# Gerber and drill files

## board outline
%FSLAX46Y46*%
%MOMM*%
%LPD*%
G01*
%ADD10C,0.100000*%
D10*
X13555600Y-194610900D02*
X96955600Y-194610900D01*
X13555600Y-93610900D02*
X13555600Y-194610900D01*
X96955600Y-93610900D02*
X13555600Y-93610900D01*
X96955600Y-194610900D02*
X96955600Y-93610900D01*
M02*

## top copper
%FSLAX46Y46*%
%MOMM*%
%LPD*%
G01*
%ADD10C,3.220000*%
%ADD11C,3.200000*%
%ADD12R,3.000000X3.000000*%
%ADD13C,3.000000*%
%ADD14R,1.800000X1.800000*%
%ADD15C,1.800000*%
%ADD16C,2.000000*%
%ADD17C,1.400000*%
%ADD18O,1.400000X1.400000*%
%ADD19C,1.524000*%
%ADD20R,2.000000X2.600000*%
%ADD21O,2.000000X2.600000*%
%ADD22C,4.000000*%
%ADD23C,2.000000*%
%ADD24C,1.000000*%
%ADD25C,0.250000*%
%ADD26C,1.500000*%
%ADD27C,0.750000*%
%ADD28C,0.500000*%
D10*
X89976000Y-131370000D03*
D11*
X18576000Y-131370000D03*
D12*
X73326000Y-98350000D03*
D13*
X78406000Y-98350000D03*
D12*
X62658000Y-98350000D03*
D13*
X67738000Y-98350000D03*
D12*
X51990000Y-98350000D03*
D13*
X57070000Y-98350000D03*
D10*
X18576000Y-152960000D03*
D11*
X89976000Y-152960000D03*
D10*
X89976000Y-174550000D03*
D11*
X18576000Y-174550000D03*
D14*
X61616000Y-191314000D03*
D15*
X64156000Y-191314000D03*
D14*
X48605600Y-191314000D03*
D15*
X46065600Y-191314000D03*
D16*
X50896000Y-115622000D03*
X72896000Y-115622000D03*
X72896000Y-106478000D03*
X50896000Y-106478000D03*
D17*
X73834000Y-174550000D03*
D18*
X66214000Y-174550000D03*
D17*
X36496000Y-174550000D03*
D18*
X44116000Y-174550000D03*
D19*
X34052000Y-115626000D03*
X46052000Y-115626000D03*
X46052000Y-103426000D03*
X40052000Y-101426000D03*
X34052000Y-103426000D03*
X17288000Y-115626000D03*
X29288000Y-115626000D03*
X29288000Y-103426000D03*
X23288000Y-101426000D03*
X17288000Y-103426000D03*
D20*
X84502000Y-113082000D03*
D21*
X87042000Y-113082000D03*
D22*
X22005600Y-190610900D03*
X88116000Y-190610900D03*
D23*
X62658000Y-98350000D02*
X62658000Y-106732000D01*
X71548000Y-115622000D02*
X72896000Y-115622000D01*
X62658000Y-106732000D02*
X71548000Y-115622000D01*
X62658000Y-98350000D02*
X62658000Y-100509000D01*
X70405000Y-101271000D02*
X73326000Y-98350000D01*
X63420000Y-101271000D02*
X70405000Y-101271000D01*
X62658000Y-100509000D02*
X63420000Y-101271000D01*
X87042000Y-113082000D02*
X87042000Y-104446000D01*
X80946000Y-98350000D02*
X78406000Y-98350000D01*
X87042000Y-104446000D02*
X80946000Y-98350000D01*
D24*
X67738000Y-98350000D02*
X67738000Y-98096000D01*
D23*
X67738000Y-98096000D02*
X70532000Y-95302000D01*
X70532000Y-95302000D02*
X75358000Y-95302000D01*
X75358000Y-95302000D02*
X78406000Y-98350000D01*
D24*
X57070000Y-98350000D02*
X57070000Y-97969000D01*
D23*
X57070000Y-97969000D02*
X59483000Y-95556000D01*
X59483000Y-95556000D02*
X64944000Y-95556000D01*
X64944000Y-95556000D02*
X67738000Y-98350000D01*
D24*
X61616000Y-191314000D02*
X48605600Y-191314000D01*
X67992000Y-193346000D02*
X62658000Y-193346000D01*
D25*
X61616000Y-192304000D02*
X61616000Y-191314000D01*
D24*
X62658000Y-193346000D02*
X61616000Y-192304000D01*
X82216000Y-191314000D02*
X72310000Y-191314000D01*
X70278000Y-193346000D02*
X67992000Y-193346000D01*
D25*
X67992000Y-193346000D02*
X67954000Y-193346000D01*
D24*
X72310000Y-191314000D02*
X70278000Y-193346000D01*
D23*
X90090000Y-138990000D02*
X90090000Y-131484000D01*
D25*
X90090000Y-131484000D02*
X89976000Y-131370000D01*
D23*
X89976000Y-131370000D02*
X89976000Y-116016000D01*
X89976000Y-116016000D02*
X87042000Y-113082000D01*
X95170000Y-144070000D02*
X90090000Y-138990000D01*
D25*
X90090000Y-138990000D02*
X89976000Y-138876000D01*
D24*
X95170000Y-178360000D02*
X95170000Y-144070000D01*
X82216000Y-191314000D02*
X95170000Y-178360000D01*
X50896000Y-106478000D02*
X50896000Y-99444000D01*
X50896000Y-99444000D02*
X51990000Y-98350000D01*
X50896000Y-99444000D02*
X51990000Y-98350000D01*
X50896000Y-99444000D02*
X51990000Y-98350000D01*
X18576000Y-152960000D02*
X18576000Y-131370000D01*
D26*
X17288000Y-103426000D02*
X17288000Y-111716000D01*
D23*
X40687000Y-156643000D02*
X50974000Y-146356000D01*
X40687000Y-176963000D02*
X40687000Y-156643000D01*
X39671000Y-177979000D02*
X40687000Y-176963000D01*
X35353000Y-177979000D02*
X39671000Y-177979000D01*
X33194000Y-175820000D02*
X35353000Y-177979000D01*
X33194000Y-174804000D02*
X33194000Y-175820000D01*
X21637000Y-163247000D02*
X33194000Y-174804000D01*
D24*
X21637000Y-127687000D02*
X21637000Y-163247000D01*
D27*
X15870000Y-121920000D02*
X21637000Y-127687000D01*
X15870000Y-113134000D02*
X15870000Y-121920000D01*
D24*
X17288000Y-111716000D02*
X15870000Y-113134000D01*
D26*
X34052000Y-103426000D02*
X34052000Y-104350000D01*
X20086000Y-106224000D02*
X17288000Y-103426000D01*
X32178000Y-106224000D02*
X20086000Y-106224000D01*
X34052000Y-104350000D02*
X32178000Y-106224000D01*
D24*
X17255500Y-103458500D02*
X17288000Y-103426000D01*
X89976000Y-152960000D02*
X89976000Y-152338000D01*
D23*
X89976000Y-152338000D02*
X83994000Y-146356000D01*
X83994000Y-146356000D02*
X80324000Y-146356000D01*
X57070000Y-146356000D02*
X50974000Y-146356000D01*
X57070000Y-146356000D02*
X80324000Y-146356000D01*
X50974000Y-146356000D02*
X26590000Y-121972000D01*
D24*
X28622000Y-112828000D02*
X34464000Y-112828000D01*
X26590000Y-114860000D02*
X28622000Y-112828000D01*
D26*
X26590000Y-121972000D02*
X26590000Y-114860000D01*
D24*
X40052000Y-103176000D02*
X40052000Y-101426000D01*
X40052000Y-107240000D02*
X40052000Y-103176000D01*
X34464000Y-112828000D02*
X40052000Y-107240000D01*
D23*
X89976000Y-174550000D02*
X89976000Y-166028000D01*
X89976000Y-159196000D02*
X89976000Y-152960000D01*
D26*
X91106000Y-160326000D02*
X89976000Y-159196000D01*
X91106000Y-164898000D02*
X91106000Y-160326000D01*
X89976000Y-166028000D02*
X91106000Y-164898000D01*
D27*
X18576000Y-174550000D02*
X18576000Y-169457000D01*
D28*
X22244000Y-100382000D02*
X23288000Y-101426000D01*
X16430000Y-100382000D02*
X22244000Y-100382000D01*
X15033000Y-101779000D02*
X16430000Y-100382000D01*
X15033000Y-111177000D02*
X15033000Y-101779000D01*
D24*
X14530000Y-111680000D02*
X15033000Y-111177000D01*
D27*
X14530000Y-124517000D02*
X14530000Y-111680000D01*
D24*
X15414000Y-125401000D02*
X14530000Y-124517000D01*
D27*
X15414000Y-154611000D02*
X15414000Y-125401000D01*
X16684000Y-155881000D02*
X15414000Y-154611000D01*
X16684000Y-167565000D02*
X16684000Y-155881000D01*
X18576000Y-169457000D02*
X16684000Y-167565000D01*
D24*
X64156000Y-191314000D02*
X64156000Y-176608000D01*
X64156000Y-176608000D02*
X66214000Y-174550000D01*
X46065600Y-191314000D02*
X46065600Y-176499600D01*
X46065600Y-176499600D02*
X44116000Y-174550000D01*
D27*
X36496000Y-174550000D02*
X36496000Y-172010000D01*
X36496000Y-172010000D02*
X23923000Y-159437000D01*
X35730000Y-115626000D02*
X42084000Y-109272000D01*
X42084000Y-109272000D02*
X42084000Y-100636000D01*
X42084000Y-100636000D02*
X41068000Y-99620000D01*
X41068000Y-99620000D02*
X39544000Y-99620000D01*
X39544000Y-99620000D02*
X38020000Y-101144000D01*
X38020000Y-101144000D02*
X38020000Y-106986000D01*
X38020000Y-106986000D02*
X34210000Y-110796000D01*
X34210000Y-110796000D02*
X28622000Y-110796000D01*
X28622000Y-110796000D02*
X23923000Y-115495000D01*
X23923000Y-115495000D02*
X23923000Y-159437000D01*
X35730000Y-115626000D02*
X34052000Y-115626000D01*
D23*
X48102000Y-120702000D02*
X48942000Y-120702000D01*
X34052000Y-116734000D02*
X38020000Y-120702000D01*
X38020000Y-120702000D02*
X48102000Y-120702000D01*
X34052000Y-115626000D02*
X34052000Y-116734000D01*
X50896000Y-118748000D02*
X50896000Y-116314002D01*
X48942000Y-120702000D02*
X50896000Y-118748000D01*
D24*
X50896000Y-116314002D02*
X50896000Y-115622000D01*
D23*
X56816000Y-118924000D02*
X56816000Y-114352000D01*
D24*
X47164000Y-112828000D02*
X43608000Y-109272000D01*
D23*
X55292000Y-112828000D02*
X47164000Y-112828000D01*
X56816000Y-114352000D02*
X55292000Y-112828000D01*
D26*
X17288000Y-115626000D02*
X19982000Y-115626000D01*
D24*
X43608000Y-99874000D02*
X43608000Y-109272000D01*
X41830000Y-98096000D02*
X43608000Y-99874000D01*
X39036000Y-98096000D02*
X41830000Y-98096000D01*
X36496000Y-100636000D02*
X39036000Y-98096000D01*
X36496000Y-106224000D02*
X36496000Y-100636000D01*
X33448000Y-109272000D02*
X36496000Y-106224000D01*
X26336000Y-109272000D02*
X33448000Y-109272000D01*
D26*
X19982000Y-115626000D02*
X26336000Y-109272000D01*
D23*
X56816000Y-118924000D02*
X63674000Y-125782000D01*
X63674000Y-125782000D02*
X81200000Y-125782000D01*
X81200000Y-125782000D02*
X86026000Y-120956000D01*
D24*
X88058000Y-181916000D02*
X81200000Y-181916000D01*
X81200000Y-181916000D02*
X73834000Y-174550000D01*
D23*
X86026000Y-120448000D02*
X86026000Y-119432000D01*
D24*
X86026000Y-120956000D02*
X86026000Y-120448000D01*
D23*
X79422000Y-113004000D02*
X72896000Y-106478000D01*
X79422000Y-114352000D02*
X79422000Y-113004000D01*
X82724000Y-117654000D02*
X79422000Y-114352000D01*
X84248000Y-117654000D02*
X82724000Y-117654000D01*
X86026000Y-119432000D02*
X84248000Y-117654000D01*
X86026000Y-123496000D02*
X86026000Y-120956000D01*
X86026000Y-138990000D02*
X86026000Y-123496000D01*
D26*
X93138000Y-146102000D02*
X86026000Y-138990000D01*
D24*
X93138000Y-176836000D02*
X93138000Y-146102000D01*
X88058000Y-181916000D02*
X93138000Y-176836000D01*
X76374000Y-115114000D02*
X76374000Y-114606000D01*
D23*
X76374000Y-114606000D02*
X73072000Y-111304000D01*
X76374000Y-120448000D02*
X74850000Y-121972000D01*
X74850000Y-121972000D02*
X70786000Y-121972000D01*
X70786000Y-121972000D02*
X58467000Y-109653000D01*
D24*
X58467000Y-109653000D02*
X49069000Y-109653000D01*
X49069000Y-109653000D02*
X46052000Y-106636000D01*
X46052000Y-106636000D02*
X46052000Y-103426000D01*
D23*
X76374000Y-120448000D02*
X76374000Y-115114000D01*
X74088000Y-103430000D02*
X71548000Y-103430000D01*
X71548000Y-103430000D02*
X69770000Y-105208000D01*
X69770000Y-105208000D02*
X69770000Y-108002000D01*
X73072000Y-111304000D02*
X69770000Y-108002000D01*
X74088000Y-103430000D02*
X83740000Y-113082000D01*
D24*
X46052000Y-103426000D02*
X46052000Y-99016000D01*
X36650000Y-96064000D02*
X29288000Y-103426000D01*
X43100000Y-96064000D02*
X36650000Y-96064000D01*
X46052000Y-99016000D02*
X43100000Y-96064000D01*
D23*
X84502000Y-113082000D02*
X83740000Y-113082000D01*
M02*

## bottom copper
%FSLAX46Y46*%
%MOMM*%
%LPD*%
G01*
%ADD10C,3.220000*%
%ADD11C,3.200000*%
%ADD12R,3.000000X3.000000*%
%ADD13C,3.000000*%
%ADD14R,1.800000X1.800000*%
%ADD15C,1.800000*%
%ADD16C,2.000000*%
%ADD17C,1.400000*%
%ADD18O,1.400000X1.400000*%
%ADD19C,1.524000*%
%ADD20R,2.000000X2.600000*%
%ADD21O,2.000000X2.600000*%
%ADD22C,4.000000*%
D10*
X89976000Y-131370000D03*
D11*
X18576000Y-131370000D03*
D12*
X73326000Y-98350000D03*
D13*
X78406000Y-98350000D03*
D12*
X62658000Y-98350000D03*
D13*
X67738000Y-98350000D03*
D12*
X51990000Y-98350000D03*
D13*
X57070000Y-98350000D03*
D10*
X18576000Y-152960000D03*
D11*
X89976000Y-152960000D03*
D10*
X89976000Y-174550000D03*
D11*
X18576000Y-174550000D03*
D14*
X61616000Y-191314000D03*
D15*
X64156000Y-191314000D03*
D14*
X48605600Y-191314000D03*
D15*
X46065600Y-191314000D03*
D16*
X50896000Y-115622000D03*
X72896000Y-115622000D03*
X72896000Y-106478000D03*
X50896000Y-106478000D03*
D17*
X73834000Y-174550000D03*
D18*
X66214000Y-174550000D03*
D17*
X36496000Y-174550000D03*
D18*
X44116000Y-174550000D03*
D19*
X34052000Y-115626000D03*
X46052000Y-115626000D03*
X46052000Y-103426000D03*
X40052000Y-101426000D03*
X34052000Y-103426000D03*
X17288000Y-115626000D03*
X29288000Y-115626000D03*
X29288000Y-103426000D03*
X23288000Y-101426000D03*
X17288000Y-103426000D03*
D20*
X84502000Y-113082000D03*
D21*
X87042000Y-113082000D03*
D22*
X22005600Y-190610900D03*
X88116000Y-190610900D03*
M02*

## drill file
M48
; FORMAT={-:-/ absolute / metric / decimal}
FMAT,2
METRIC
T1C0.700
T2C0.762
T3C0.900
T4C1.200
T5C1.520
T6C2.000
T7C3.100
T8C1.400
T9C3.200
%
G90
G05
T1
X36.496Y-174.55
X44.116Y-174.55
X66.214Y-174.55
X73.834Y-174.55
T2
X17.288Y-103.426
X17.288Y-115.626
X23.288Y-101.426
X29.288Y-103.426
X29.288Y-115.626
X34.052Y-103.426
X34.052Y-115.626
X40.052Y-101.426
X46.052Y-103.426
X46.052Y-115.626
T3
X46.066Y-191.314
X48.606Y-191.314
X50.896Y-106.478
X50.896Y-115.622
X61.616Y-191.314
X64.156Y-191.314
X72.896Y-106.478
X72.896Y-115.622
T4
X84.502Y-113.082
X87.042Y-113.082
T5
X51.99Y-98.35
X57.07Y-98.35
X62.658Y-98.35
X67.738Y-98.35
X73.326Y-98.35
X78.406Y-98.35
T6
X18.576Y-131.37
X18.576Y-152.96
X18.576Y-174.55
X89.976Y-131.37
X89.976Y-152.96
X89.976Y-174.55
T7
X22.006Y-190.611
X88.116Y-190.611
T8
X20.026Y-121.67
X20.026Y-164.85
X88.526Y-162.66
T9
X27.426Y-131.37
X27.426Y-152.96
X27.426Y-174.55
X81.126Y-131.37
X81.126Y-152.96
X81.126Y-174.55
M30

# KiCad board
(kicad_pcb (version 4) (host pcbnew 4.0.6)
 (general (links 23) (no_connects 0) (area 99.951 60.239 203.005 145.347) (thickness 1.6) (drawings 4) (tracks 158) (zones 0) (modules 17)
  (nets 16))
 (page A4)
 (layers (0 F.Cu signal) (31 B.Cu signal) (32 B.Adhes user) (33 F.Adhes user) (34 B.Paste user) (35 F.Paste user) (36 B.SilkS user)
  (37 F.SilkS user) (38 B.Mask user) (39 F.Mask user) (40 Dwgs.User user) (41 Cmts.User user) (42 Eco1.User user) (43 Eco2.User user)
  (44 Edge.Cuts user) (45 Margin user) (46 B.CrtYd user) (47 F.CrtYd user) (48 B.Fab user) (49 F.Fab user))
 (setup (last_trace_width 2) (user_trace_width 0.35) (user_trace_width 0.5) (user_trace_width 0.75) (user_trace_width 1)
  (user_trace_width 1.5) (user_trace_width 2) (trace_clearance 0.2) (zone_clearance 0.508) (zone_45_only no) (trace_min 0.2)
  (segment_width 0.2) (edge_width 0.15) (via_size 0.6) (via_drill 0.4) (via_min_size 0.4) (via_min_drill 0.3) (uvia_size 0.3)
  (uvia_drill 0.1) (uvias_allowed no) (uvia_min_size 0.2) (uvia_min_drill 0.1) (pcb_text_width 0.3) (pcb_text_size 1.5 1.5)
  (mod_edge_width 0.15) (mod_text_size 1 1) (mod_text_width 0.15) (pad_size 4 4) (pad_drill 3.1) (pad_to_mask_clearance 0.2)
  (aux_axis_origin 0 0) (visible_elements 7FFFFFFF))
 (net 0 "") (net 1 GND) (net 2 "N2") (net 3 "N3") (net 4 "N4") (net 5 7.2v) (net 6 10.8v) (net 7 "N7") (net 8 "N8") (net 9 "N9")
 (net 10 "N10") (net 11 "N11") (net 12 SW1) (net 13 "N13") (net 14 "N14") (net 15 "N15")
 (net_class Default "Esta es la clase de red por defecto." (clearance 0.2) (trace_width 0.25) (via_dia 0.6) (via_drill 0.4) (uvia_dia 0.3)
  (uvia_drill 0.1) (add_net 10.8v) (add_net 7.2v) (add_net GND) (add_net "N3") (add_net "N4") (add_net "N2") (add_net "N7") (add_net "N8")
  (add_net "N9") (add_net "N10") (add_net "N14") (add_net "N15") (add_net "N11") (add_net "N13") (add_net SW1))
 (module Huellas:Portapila (layer F.Cu) (at 54.276 131.37 180)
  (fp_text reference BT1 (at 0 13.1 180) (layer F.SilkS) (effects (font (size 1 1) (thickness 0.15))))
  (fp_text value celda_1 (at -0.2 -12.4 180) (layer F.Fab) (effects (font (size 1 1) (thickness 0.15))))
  (pad "" np_thru_hole circle (at 34.25 9.7 180) (size 1.4 1.4) (drill 1.4) (layers *.Cu *.Mask F.SilkS))
  (pad 2 thru_hole circle (at -35.7 0 180) (size 3.22 3.22) (drill 2) (layers *.Cu *.Mask F.SilkS) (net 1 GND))
  (pad 1 thru_hole circle (at 35.7 0 180) (size 3.2 3.2) (drill 2) (layers *.Cu *.Mask F.SilkS) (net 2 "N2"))
  (pad "" np_thru_hole circle (at 26.85 0 180) (size 3.2 3.2) (drill 3.2) (layers *.Cu *.Mask F.SilkS))
  (pad "" np_thru_hole circle (at -26.85 0 180) (size 3.2 3.2) (drill 3.2) (layers *.Cu *.Mask F.SilkS)))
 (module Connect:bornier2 (layer F.Cu) (at 73.326 98.35)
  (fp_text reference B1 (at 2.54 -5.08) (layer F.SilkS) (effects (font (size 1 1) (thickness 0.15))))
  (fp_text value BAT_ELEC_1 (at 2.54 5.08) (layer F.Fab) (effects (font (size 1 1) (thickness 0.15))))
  (pad 1 thru_hole rect (at 0 0) (size 3 3) (drill 1.52) (layers *.Cu *.Mask) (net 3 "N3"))
  (pad 2 thru_hole circle (at 5.08 0) (size 3 3) (drill 1.52) (layers *.Cu *.Mask) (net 1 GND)))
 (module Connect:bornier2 (layer F.Cu) (at 62.658 98.35)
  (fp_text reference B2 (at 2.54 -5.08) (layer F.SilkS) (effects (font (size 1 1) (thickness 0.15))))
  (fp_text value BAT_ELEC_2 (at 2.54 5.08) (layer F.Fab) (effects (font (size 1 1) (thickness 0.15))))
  (pad 1 thru_hole rect (at 0 0) (size 3 3) (drill 1.52) (layers *.Cu *.Mask) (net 3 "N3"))
  (pad 2 thru_hole circle (at 5.08 0) (size 3 3) (drill 1.52) (layers *.Cu *.Mask) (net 1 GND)))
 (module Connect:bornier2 (layer F.Cu) (at 51.99 98.35)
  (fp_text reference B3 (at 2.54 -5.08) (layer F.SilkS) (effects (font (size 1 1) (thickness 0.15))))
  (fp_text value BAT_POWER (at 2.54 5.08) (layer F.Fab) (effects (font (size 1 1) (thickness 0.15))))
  (pad 1 thru_hole rect (at 0 0) (size 3 3) (drill 1.52) (layers *.Cu *.Mask) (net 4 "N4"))
  (pad 2 thru_hole circle (at 5.08 0) (size 3 3) (drill 1.52) (layers *.Cu *.Mask) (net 1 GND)))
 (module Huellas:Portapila (layer F.Cu) (at 54.276 152.96)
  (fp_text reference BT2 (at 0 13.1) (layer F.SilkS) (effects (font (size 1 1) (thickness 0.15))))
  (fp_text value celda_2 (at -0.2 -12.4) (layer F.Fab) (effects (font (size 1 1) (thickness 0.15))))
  (pad "" np_thru_hole circle (at 34.25 9.7) (size 1.4 1.4) (drill 1.4) (layers *.Cu *.Mask F.SilkS))
  (pad 2 thru_hole circle (at -35.7 0) (size 3.22 3.22) (drill 2) (layers *.Cu *.Mask F.SilkS) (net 2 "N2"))
  (pad 1 thru_hole circle (at 35.7 0) (size 3.2 3.2) (drill 2) (layers *.Cu *.Mask F.SilkS) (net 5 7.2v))
  (pad "" np_thru_hole circle (at 26.85 0) (size 3.2 3.2) (drill 3.2) (layers *.Cu *.Mask F.SilkS))
  (pad "" np_thru_hole circle (at -26.85 0) (size 3.2 3.2) (drill 3.2) (layers *.Cu *.Mask F.SilkS)))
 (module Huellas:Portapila (layer F.Cu) (at 54.276 174.55 180)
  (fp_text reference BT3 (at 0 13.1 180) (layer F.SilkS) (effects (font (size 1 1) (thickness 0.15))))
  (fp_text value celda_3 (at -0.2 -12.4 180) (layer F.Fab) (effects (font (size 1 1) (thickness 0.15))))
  (pad "" np_thru_hole circle (at 34.25 9.7 180) (size 1.4 1.4) (drill 1.4) (layers *.Cu *.Mask F.SilkS))
  (pad 2 thru_hole circle (at -35.7 0 180) (size 3.22 3.22) (drill 2) (layers *.Cu *.Mask F.SilkS) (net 5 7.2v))
  (pad 1 thru_hole circle (at 35.7 0 180) (size 3.2 3.2) (drill 2) (layers *.Cu *.Mask F.SilkS) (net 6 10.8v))
  (pad "" np_thru_hole circle (at 26.85 0 180) (size 3.2 3.2) (drill 3.2) (layers *.Cu *.Mask F.SilkS))
  (pad "" np_thru_hole circle (at -26.85 0 180) (size 3.2 3.2) (drill 3.2) (layers *.Cu *.Mask F.SilkS)))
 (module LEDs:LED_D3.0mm (layer F.Cu) (at 61.616 191.314)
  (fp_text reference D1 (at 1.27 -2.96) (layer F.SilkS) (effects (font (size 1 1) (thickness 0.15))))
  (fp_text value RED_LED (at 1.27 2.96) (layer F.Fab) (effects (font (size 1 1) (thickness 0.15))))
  (pad 1 thru_hole rect (at 0 0) (size 1.8 1.8) (drill 0.9) (layers *.Cu *.Mask) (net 1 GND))
  (pad 2 thru_hole circle (at 2.54 0) (size 1.8 1.8) (drill 0.9) (layers *.Cu *.Mask) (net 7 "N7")))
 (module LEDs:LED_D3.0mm (layer F.Cu) (at 48.6056 191.314 180)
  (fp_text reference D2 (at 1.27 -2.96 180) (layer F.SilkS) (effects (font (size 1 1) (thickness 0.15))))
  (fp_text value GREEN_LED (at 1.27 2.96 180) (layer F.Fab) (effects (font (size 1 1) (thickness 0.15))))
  (pad 1 thru_hole rect (at 0 0 180) (size 1.8 1.8) (drill 0.9) (layers *.Cu *.Mask) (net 1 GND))
  (pad 2 thru_hole circle (at 2.54 0 180) (size 1.8 1.8) (drill 0.9) (layers *.Cu *.Mask) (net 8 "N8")))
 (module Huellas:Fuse (layer F.Cu) (at 61.896 115.622 90)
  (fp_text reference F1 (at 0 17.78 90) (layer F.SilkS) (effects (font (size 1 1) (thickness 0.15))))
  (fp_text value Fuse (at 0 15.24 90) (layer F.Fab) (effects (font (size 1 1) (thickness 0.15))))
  (pad 2 thru_hole circle (at 0 -11 90) (size 2 2) (drill 0.9) (layers *.Cu *.Mask) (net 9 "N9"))
  (pad 1 thru_hole circle (at 0 11 90) (size 2 2) (drill 0.9) (layers *.Cu *.Mask) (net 3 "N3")))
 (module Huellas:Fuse (layer F.Cu) (at 61.896 106.478 270)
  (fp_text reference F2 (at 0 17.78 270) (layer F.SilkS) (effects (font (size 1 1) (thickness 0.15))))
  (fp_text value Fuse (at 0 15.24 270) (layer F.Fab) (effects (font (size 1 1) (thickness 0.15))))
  (pad 2 thru_hole circle (at 0 -11 270) (size 2 2) (drill 0.9) (layers *.Cu *.Mask) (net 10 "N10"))
  (pad 1 thru_hole circle (at 0 11 270) (size 2 2) (drill 0.9) (layers *.Cu *.Mask) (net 4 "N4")))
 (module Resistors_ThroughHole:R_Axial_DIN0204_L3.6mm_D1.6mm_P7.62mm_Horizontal (layer F.Cu) (at 73.834 174.55 180)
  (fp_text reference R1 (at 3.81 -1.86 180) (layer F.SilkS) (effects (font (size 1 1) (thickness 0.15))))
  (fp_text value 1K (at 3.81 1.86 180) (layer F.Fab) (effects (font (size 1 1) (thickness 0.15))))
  (pad 1 thru_hole circle (at 0 0 180) (size 1.4 1.4) (drill 0.7) (layers *.Cu *.Mask) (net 10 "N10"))
  (pad 2 thru_hole oval (at 7.62 0 180) (size 1.4 1.4) (drill 0.7) (layers *.Cu *.Mask) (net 7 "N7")))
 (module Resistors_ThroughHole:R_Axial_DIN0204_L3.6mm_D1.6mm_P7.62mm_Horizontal (layer F.Cu) (at 36.496 174.55)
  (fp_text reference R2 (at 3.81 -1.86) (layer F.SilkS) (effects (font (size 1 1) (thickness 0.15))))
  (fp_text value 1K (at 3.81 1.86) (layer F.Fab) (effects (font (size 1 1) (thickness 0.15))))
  (pad 1 thru_hole circle (at 0 0) (size 1.4 1.4) (drill 0.7) (layers *.Cu *.Mask) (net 9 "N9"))
  (pad 2 thru_hole oval (at 7.62 0) (size 1.4 1.4) (drill 0.7) (layers *.Cu *.Mask) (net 8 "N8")))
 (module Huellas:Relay (layer F.Cu) (at 40.052 109.526 180)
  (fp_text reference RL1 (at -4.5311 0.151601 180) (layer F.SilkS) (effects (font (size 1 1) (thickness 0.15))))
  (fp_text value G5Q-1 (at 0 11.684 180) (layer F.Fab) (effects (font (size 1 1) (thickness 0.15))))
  (pad 3 thru_hole circle (at 6 -6.1 180) (size 1.524 1.524) (drill 0.762) (layers *.Cu *.Mask) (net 9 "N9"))
  (pad 4 thru_hole circle (at -6 -6.1 180) (size 1.524 1.524) (drill 0.762) (layers *.Cu *.Mask) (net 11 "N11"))
  (pad 1 thru_hole circle (at -6 6.1 180) (size 1.524 1.524) (drill 0.762) (layers *.Cu *.Mask) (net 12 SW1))
  (pad 2 thru_hole circle (at 0 8.1 180) (size 1.524 1.524) (drill 0.762) (layers *.Cu *.Mask) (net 5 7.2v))
  (pad 5 thru_hole circle (at 6 6.1 180) (size 1.524 1.524) (drill 0.762) (layers *.Cu *.Mask) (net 5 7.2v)))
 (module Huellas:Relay (layer F.Cu) (at 23.288 109.526 180)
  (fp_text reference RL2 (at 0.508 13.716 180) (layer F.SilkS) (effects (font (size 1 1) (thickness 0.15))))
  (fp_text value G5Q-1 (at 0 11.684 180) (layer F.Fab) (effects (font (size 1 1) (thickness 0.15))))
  (pad 3 thru_hole circle (at 6 -6.1 180) (size 1.524 1.524) (drill 0.762) (layers *.Cu *.Mask) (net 10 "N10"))
  (pad 4 thru_hole circle (at -6 -6.1 180) (size 1.524 1.524) (drill 0.762) (layers *.Cu *.Mask) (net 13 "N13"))
  (pad 1 thru_hole circle (at -6 6.1 180) (size 1.524 1.524) (drill 0.762) (layers *.Cu *.Mask) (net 12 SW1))
  (pad 2 thru_hole circle (at 0 8.1 180) (size 1.524 1.524) (drill 0.762) (layers *.Cu *.Mask) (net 6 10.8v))
  (pad 5 thru_hole circle (at 6 6.1 180) (size 1.524 1.524) (drill 0.762) (layers *.Cu *.Mask) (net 5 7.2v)))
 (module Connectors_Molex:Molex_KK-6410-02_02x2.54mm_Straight (layer F.Cu) (at 84.502 113.082)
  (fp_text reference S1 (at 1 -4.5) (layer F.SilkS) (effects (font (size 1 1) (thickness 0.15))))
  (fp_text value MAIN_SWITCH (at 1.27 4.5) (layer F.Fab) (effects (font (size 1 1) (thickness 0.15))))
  (pad 1 thru_hole rect (at 0 0) (size 2 2.6) (drill 1.2) (layers *.Cu *.Mask) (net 12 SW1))
  (pad 2 thru_hole oval (at 2.54 0) (size 2 2.6) (drill 1.2) (layers *.Cu *.Mask) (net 1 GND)))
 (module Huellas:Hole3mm (layer F.Cu) (at 16.684 191.314 90)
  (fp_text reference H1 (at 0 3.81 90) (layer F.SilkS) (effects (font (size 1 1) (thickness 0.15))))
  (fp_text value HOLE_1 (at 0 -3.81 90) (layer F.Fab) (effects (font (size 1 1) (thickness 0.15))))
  (pad 1 thru_hole circle (at 0.7031 5.3216 90) (size 4 4) (drill 3.1) (layers *.Cu *.Mask) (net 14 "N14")))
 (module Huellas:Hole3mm (layer F.Cu) (at 92.122 190.298 90)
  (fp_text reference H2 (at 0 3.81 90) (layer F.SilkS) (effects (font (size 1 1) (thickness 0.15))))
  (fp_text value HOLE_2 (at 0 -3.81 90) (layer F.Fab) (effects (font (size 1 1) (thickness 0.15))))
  (pad 1 thru_hole circle (at -0.3129 -4.006 90) (size 4 4) (drill 3.1) (layers *.Cu *.Mask) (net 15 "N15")))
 (gr_line (start 13.5556 194.6109) (end 96.9556 194.6109) (layer Edge.Cuts) (width 0.1))
 (gr_line (start 13.5556 93.6109) (end 13.5556 194.6109) (layer Edge.Cuts) (width 0.1))
 (gr_line (start 96.9556 93.6109) (end 13.5556 93.6109) (layer Edge.Cuts) (width 0.1))
 (gr_line (start 96.9556 194.6109) (end 96.9556 93.6109) (layer Edge.Cuts) (width 0.1))
 (segment (start 62.658 98.35) (end 62.658 106.732) (width 2) (layer F.Cu) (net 3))
 (segment (start 71.548 115.622) (end 72.896 115.622) (width 2) (layer F.Cu) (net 3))
 (segment (start 62.658 106.732) (end 71.548 115.622) (width 2) (layer F.Cu) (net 3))
 (segment (start 62.658 98.35) (end 62.658 100.509) (width 2) (layer F.Cu) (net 3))
 (segment (start 70.405 101.271) (end 73.326 98.35) (width 2) (layer F.Cu) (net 3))
 (segment (start 63.42 101.271) (end 70.405 101.271) (width 2) (layer F.Cu) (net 3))
 (segment (start 62.658 100.509) (end 63.42 101.271) (width 2) (layer F.Cu) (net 3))
 (segment (start 87.042 113.082) (end 87.042 104.446) (width 2) (layer F.Cu) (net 1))
 (segment (start 80.946 98.35) (end 78.406 98.35) (width 2) (layer F.Cu) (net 1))
 (segment (start 87.042 104.446) (end 80.946 98.35) (width 2) (layer F.Cu) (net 1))
 (segment (start 67.738 98.35) (end 67.738 98.096) (width 1) (layer F.Cu) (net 1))
 (segment (start 67.738 98.096) (end 70.532 95.302) (width 2) (layer F.Cu) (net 1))
 (segment (start 70.532 95.302) (end 75.358 95.302) (width 2) (layer F.Cu) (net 1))
 (segment (start 75.358 95.302) (end 78.406 98.35) (width 2) (layer F.Cu) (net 1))
 (segment (start 57.07 98.35) (end 57.07 97.969) (width 1) (layer F.Cu) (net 1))
 (segment (start 57.07 97.969) (end 59.483 95.556) (width 2) (layer F.Cu) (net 1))
 (segment (start 59.483 95.556) (end 64.944 95.556) (width 2) (layer F.Cu) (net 1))
 (segment (start 64.944 95.556) (end 67.738 98.35) (width 2) (layer F.Cu) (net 1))
 (segment (start 61.616 191.314) (end 48.6056 191.314) (width 1) (layer F.Cu) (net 1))
 (segment (start 67.992 193.346) (end 62.658 193.346) (width 1) (layer F.Cu) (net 1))
 (segment (start 61.616 192.304) (end 61.616 191.314) (width 0.25) (layer F.Cu) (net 1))
 (segment (start 62.658 193.346) (end 61.616 192.304) (width 1) (layer F.Cu) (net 1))
 (segment (start 82.216 191.314) (end 72.31 191.314) (width 1) (layer F.Cu) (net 1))
 (segment (start 70.278 193.346) (end 67.992 193.346) (width 1) (layer F.Cu) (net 1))
 (segment (start 67.992 193.346) (end 67.954 193.346) (width 0.25) (layer F.Cu) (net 1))
 (segment (start 72.31 191.314) (end 70.278 193.346) (width 1) (layer F.Cu) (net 1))
 (segment (start 90.09 138.99) (end 90.09 131.484) (width 2) (layer F.Cu) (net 1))
 (segment (start 90.09 131.484) (end 89.976 131.37) (width 0.25) (layer F.Cu) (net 1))
 (segment (start 89.976 131.37) (end 89.976 116.016) (width 2) (layer F.Cu) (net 1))
 (segment (start 89.976 116.016) (end 87.042 113.082) (width 2) (layer F.Cu) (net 1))
 (segment (start 95.17 144.07) (end 90.09 138.99) (width 2) (layer F.Cu) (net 1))
 (segment (start 90.09 138.99) (end 89.976 138.876) (width 0.25) (layer F.Cu) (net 1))
 (segment (start 95.17 178.36) (end 95.17 144.07) (width 1) (layer F.Cu) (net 1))
 (segment (start 82.216 191.314) (end 95.17 178.36) (width 1) (layer F.Cu) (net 1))
 (segment (start 50.896 106.478) (end 50.896 99.444) (width 1) (layer F.Cu) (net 4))
 (segment (start 50.896 99.444) (end 51.99 98.35) (width 1) (layer F.Cu) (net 4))
 (segment (start 50.896 99.444) (end 51.99 98.35) (width 1) (layer F.Cu) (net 4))
 (segment (start 50.896 99.444) (end 51.99 98.35) (width 1) (layer F.Cu) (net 4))
 (segment (start 18.576 152.96) (end 18.576 131.37) (width 1) (layer F.Cu) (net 2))
 (segment (start 17.288 103.426) (end 17.288 111.716) (width 1.5) (layer F.Cu) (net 5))
 (segment (start 40.687 156.643) (end 50.974 146.356) (width 2) (layer F.Cu) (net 5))
 (segment (start 40.687 176.963) (end 40.687 156.643) (width 2) (layer F.Cu) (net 5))
 (segment (start 39.671 177.979) (end 40.687 176.963) (width 2) (layer F.Cu) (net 5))
 (segment (start 35.353 177.979) (end 39.671 177.979) (width 2) (layer F.Cu) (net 5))
 (segment (start 33.194 175.82) (end 35.353 177.979) (width 2) (layer F.Cu) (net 5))
 (segment (start 33.194 174.804) (end 33.194 175.82) (width 2) (layer F.Cu) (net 5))
 (segment (start 21.637 163.247) (end 33.194 174.804) (width 2) (layer F.Cu) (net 5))
 (segment (start 21.637 127.687) (end 21.637 163.247) (width 1) (layer F.Cu) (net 5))
 (segment (start 15.87 121.92) (end 21.637 127.687) (width 0.75) (layer F.Cu) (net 5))
 (segment (start 15.87 113.134) (end 15.87 121.92) (width 0.75) (layer F.Cu) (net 5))
 (segment (start 17.288 111.716) (end 15.87 113.134) (width 1) (layer F.Cu) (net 5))
 (segment (start 34.052 103.426) (end 34.052 104.35) (width 1.5) (layer F.Cu) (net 5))
 (segment (start 20.086 106.224) (end 17.288 103.426) (width 1.5) (layer F.Cu) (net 5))
 (segment (start 32.178 106.224) (end 20.086 106.224) (width 1.5) (layer F.Cu) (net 5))
 (segment (start 34.052 104.35) (end 32.178 106.224) (width 1.5) (layer F.Cu) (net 5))
 (segment (start 17.2555 103.4585) (end 17.288 103.426) (width 1) (layer F.Cu) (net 5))
 (segment (start 89.976 152.96) (end 89.976 152.338) (width 1) (layer F.Cu) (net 5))
 (segment (start 89.976 152.338) (end 83.994 146.356) (width 2) (layer F.Cu) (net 5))
 (segment (start 83.994 146.356) (end 80.324 146.356) (width 2) (layer F.Cu) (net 5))
 (segment (start 57.07 146.356) (end 50.974 146.356) (width 2) (layer F.Cu) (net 5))
 (segment (start 57.07 146.356) (end 80.324 146.356) (width 2) (layer F.Cu) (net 5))
 (segment (start 50.974 146.356) (end 26.59 121.972) (width 2) (layer F.Cu) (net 5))
 (segment (start 28.622 112.828) (end 34.464 112.828) (width 1) (layer F.Cu) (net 5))
 (segment (start 26.59 114.86) (end 28.622 112.828) (width 1) (layer F.Cu) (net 5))
 (segment (start 26.59 121.972) (end 26.59 114.86) (width 1.5) (layer F.Cu) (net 5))
 (segment (start 40.052 103.176) (end 40.052 101.426) (width 1) (layer F.Cu) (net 5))
 (segment (start 40.052 107.24) (end 40.052 103.176) (width 1) (layer F.Cu) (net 5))
 (segment (start 34.464 112.828) (end 40.052 107.24) (width 1) (layer F.Cu) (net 5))
 (segment (start 89.976 174.55) (end 89.976 166.028) (width 2) (layer F.Cu) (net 5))
 (segment (start 89.976 159.196) (end 89.976 152.96) (width 2) (layer F.Cu) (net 5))
 (segment (start 91.106 160.326) (end 89.976 159.196) (width 1.5) (layer F.Cu) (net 5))
 (segment (start 91.106 164.898) (end 91.106 160.326) (width 1.5) (layer F.Cu) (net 5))
 (segment (start 89.976 166.028) (end 91.106 164.898) (width 1.5) (layer F.Cu) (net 5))
 (segment (start 18.576 174.55) (end 18.576 169.457) (width 0.75) (layer F.Cu) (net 6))
 (segment (start 22.244 100.382) (end 23.288 101.426) (width 0.5) (layer F.Cu) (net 6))
 (segment (start 16.43 100.382) (end 22.244 100.382) (width 0.5) (layer F.Cu) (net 6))
 (segment (start 15.033 101.779) (end 16.43 100.382) (width 0.5) (layer F.Cu) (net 6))
 (segment (start 15.033 111.177) (end 15.033 101.779) (width 0.5) (layer F.Cu) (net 6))
 (segment (start 14.53 111.68) (end 15.033 111.177) (width 1) (layer F.Cu) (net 6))
 (segment (start 14.53 124.517) (end 14.53 111.68) (width 0.75) (layer F.Cu) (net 6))
 (segment (start 15.414 125.401) (end 14.53 124.517) (width 1) (layer F.Cu) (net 6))
 (segment (start 15.414 154.611) (end 15.414 125.401) (width 0.75) (layer F.Cu) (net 6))
 (segment (start 16.684 155.881) (end 15.414 154.611) (width 0.75) (layer F.Cu) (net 6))
 (segment (start 16.684 167.565) (end 16.684 155.881) (width 0.75) (layer F.Cu) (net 6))
 (segment (start 18.576 169.457) (end 16.684 167.565) (width 0.75) (layer F.Cu) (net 6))
 (segment (start 64.156 191.314) (end 64.156 176.608) (width 1) (layer F.Cu) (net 7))
 (segment (start 64.156 176.608) (end 66.214 174.55) (width 1) (layer F.Cu) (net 7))
 (segment (start 46.0656 191.314) (end 46.0656 176.4996) (width 1) (layer F.Cu) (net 8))
 (segment (start 46.0656 176.4996) (end 44.116 174.55) (width 1) (layer F.Cu) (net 8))
 (segment (start 36.496 174.55) (end 36.496 172.01) (width 0.75) (layer F.Cu) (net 9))
 (segment (start 36.496 172.01) (end 23.923 159.437) (width 0.75) (layer F.Cu) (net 9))
 (segment (start 35.73 115.626) (end 42.084 109.272) (width 0.75) (layer F.Cu) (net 9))
 (segment (start 42.084 109.272) (end 42.084 100.636) (width 0.75) (layer F.Cu) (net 9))
 (segment (start 42.084 100.636) (end 41.068 99.62) (width 0.75) (layer F.Cu) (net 9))
 (segment (start 41.068 99.62) (end 39.544 99.62) (width 0.75) (layer F.Cu) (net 9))
 (segment (start 39.544 99.62) (end 38.02 101.144) (width 0.75) (layer F.Cu) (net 9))
 (segment (start 38.02 101.144) (end 38.02 106.986) (width 0.75) (layer F.Cu) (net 9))
 (segment (start 38.02 106.986) (end 34.21 110.796) (width 0.75) (layer F.Cu) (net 9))
 (segment (start 34.21 110.796) (end 28.622 110.796) (width 0.75) (layer F.Cu) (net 9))
 (segment (start 28.622 110.796) (end 23.923 115.495) (width 0.75) (layer F.Cu) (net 9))
 (segment (start 23.923 115.495) (end 23.923 159.437) (width 0.75) (layer F.Cu) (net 9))
 (segment (start 35.73 115.626) (end 34.052 115.626) (width 0.75) (layer F.Cu) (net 9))
 (segment (start 48.102 120.702) (end 48.942 120.702) (width 2) (layer F.Cu) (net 9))
 (segment (start 34.052 116.734) (end 38.02 120.702) (width 2) (layer F.Cu) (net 9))
 (segment (start 38.02 120.702) (end 48.102 120.702) (width 2) (layer F.Cu) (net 9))
 (segment (start 34.052 115.626) (end 34.052 116.734) (width 2) (layer F.Cu) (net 9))
 (segment (start 50.896 118.748) (end 50.896 116.314002) (width 2) (layer F.Cu) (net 9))
 (segment (start 48.942 120.702) (end 50.896 118.748) (width 2) (layer F.Cu) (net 9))
 (segment (start 50.896 116.314002) (end 50.896 115.622) (width 1) (layer F.Cu) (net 9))
 (segment (start 56.816 118.924) (end 56.816 114.352) (width 2) (layer F.Cu) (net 10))
 (segment (start 47.164 112.828) (end 43.608 109.272) (width 1) (layer F.Cu) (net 10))
 (segment (start 55.292 112.828) (end 47.164 112.828) (width 2) (layer F.Cu) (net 10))
 (segment (start 56.816 114.352) (end 55.292 112.828) (width 2) (layer F.Cu) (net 10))
 (segment (start 17.288 115.626) (end 19.982 115.626) (width 1.5) (layer F.Cu) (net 10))
 (segment (start 43.608 99.874) (end 43.608 109.272) (width 1) (layer F.Cu) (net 10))
 (segment (start 41.83 98.096) (end 43.608 99.874) (width 1) (layer F.Cu) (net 10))
 (segment (start 39.036 98.096) (end 41.83 98.096) (width 1) (layer F.Cu) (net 10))
 (segment (start 36.496 100.636) (end 39.036 98.096) (width 1) (layer F.Cu) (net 10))
 (segment (start 36.496 106.224) (end 36.496 100.636) (width 1) (layer F.Cu) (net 10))
 (segment (start 33.448 109.272) (end 36.496 106.224) (width 1) (layer F.Cu) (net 10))
 (segment (start 26.336 109.272) (end 33.448 109.272) (width 1) (layer F.Cu) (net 10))
 (segment (start 19.982 115.626) (end 26.336 109.272) (width 1.5) (layer F.Cu) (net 10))
 (segment (start 56.816 118.924) (end 63.674 125.782) (width 2) (layer F.Cu) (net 10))
 (segment (start 63.674 125.782) (end 81.2 125.782) (width 2) (layer F.Cu) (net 10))
 (segment (start 81.2 125.782) (end 86.026 120.956) (width 2) (layer F.Cu) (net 10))
 (segment (start 88.058 181.916) (end 81.2 181.916) (width 1) (layer F.Cu) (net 10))
 (segment (start 81.2 181.916) (end 73.834 174.55) (width 1) (layer F.Cu) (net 10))
 (segment (start 86.026 120.448) (end 86.026 119.432) (width 2) (layer F.Cu) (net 10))
 (segment (start 86.026 120.956) (end 86.026 120.448) (width 1) (layer F.Cu) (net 10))
 (segment (start 79.422 113.004) (end 72.896 106.478) (width 2) (layer F.Cu) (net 10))
 (segment (start 79.422 114.352) (end 79.422 113.004) (width 2) (layer F.Cu) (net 10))
 (segment (start 82.724 117.654) (end 79.422 114.352) (width 2) (layer F.Cu) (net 10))
 (segment (start 84.248 117.654) (end 82.724 117.654) (width 2) (layer F.Cu) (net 10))
 (segment (start 86.026 119.432) (end 84.248 117.654) (width 2) (layer F.Cu) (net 10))
 (segment (start 86.026 123.496) (end 86.026 120.956) (width 2) (layer F.Cu) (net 10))
 (segment (start 86.026 138.99) (end 86.026 123.496) (width 2) (layer F.Cu) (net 10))
 (segment (start 93.138 146.102) (end 86.026 138.99) (width 1.5) (layer F.Cu) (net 10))
 (segment (start 93.138 176.836) (end 93.138 146.102) (width 1) (layer F.Cu) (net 10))
 (segment (start 88.058 181.916) (end 93.138 176.836) (width 1) (layer F.Cu) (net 10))
 (segment (start 76.374 115.114) (end 76.374 114.606) (width 1) (layer F.Cu) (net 12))
 (segment (start 76.374 114.606) (end 73.072 111.304) (width 2) (layer F.Cu) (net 12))
 (segment (start 76.374 120.448) (end 74.85 121.972) (width 2) (layer F.Cu) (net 12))
 (segment (start 74.85 121.972) (end 70.786 121.972) (width 2) (layer F.Cu) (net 12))
 (segment (start 70.786 121.972) (end 58.467 109.653) (width 2) (layer F.Cu) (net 12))
 (segment (start 58.467 109.653) (end 49.069 109.653) (width 1) (layer F.Cu) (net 12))
 (segment (start 49.069 109.653) (end 46.052 106.636) (width 1) (layer F.Cu) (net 12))
 (segment (start 46.052 106.636) (end 46.052 103.426) (width 1) (layer F.Cu) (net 12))
 (segment (start 76.374 120.448) (end 76.374 115.114) (width 2) (layer F.Cu) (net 12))
 (segment (start 74.088 103.43) (end 71.548 103.43) (width 2) (layer F.Cu) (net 12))
 (segment (start 71.548 103.43) (end 69.77 105.208) (width 2) (layer F.Cu) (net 12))
 (segment (start 69.77 105.208) (end 69.77 108.002) (width 2) (layer F.Cu) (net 12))
 (segment (start 73.072 111.304) (end 69.77 108.002) (width 2) (layer F.Cu) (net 12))
 (segment (start 74.088 103.43) (end 83.74 113.082) (width 2) (layer F.Cu) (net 12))
 (segment (start 46.052 103.426) (end 46.052 99.016) (width 1) (layer F.Cu) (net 12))
 (segment (start 36.65 96.064) (end 29.288 103.426) (width 1) (layer F.Cu) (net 12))
 (segment (start 43.1 96.064) (end 36.65 96.064) (width 1) (layer F.Cu) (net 12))
 (segment (start 46.052 99.016) (end 43.1 96.064) (width 1) (layer F.Cu) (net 12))
 (segment (start 84.502 113.082) (end 83.74 113.082) (width 2) (layer F.Cu) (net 12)))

